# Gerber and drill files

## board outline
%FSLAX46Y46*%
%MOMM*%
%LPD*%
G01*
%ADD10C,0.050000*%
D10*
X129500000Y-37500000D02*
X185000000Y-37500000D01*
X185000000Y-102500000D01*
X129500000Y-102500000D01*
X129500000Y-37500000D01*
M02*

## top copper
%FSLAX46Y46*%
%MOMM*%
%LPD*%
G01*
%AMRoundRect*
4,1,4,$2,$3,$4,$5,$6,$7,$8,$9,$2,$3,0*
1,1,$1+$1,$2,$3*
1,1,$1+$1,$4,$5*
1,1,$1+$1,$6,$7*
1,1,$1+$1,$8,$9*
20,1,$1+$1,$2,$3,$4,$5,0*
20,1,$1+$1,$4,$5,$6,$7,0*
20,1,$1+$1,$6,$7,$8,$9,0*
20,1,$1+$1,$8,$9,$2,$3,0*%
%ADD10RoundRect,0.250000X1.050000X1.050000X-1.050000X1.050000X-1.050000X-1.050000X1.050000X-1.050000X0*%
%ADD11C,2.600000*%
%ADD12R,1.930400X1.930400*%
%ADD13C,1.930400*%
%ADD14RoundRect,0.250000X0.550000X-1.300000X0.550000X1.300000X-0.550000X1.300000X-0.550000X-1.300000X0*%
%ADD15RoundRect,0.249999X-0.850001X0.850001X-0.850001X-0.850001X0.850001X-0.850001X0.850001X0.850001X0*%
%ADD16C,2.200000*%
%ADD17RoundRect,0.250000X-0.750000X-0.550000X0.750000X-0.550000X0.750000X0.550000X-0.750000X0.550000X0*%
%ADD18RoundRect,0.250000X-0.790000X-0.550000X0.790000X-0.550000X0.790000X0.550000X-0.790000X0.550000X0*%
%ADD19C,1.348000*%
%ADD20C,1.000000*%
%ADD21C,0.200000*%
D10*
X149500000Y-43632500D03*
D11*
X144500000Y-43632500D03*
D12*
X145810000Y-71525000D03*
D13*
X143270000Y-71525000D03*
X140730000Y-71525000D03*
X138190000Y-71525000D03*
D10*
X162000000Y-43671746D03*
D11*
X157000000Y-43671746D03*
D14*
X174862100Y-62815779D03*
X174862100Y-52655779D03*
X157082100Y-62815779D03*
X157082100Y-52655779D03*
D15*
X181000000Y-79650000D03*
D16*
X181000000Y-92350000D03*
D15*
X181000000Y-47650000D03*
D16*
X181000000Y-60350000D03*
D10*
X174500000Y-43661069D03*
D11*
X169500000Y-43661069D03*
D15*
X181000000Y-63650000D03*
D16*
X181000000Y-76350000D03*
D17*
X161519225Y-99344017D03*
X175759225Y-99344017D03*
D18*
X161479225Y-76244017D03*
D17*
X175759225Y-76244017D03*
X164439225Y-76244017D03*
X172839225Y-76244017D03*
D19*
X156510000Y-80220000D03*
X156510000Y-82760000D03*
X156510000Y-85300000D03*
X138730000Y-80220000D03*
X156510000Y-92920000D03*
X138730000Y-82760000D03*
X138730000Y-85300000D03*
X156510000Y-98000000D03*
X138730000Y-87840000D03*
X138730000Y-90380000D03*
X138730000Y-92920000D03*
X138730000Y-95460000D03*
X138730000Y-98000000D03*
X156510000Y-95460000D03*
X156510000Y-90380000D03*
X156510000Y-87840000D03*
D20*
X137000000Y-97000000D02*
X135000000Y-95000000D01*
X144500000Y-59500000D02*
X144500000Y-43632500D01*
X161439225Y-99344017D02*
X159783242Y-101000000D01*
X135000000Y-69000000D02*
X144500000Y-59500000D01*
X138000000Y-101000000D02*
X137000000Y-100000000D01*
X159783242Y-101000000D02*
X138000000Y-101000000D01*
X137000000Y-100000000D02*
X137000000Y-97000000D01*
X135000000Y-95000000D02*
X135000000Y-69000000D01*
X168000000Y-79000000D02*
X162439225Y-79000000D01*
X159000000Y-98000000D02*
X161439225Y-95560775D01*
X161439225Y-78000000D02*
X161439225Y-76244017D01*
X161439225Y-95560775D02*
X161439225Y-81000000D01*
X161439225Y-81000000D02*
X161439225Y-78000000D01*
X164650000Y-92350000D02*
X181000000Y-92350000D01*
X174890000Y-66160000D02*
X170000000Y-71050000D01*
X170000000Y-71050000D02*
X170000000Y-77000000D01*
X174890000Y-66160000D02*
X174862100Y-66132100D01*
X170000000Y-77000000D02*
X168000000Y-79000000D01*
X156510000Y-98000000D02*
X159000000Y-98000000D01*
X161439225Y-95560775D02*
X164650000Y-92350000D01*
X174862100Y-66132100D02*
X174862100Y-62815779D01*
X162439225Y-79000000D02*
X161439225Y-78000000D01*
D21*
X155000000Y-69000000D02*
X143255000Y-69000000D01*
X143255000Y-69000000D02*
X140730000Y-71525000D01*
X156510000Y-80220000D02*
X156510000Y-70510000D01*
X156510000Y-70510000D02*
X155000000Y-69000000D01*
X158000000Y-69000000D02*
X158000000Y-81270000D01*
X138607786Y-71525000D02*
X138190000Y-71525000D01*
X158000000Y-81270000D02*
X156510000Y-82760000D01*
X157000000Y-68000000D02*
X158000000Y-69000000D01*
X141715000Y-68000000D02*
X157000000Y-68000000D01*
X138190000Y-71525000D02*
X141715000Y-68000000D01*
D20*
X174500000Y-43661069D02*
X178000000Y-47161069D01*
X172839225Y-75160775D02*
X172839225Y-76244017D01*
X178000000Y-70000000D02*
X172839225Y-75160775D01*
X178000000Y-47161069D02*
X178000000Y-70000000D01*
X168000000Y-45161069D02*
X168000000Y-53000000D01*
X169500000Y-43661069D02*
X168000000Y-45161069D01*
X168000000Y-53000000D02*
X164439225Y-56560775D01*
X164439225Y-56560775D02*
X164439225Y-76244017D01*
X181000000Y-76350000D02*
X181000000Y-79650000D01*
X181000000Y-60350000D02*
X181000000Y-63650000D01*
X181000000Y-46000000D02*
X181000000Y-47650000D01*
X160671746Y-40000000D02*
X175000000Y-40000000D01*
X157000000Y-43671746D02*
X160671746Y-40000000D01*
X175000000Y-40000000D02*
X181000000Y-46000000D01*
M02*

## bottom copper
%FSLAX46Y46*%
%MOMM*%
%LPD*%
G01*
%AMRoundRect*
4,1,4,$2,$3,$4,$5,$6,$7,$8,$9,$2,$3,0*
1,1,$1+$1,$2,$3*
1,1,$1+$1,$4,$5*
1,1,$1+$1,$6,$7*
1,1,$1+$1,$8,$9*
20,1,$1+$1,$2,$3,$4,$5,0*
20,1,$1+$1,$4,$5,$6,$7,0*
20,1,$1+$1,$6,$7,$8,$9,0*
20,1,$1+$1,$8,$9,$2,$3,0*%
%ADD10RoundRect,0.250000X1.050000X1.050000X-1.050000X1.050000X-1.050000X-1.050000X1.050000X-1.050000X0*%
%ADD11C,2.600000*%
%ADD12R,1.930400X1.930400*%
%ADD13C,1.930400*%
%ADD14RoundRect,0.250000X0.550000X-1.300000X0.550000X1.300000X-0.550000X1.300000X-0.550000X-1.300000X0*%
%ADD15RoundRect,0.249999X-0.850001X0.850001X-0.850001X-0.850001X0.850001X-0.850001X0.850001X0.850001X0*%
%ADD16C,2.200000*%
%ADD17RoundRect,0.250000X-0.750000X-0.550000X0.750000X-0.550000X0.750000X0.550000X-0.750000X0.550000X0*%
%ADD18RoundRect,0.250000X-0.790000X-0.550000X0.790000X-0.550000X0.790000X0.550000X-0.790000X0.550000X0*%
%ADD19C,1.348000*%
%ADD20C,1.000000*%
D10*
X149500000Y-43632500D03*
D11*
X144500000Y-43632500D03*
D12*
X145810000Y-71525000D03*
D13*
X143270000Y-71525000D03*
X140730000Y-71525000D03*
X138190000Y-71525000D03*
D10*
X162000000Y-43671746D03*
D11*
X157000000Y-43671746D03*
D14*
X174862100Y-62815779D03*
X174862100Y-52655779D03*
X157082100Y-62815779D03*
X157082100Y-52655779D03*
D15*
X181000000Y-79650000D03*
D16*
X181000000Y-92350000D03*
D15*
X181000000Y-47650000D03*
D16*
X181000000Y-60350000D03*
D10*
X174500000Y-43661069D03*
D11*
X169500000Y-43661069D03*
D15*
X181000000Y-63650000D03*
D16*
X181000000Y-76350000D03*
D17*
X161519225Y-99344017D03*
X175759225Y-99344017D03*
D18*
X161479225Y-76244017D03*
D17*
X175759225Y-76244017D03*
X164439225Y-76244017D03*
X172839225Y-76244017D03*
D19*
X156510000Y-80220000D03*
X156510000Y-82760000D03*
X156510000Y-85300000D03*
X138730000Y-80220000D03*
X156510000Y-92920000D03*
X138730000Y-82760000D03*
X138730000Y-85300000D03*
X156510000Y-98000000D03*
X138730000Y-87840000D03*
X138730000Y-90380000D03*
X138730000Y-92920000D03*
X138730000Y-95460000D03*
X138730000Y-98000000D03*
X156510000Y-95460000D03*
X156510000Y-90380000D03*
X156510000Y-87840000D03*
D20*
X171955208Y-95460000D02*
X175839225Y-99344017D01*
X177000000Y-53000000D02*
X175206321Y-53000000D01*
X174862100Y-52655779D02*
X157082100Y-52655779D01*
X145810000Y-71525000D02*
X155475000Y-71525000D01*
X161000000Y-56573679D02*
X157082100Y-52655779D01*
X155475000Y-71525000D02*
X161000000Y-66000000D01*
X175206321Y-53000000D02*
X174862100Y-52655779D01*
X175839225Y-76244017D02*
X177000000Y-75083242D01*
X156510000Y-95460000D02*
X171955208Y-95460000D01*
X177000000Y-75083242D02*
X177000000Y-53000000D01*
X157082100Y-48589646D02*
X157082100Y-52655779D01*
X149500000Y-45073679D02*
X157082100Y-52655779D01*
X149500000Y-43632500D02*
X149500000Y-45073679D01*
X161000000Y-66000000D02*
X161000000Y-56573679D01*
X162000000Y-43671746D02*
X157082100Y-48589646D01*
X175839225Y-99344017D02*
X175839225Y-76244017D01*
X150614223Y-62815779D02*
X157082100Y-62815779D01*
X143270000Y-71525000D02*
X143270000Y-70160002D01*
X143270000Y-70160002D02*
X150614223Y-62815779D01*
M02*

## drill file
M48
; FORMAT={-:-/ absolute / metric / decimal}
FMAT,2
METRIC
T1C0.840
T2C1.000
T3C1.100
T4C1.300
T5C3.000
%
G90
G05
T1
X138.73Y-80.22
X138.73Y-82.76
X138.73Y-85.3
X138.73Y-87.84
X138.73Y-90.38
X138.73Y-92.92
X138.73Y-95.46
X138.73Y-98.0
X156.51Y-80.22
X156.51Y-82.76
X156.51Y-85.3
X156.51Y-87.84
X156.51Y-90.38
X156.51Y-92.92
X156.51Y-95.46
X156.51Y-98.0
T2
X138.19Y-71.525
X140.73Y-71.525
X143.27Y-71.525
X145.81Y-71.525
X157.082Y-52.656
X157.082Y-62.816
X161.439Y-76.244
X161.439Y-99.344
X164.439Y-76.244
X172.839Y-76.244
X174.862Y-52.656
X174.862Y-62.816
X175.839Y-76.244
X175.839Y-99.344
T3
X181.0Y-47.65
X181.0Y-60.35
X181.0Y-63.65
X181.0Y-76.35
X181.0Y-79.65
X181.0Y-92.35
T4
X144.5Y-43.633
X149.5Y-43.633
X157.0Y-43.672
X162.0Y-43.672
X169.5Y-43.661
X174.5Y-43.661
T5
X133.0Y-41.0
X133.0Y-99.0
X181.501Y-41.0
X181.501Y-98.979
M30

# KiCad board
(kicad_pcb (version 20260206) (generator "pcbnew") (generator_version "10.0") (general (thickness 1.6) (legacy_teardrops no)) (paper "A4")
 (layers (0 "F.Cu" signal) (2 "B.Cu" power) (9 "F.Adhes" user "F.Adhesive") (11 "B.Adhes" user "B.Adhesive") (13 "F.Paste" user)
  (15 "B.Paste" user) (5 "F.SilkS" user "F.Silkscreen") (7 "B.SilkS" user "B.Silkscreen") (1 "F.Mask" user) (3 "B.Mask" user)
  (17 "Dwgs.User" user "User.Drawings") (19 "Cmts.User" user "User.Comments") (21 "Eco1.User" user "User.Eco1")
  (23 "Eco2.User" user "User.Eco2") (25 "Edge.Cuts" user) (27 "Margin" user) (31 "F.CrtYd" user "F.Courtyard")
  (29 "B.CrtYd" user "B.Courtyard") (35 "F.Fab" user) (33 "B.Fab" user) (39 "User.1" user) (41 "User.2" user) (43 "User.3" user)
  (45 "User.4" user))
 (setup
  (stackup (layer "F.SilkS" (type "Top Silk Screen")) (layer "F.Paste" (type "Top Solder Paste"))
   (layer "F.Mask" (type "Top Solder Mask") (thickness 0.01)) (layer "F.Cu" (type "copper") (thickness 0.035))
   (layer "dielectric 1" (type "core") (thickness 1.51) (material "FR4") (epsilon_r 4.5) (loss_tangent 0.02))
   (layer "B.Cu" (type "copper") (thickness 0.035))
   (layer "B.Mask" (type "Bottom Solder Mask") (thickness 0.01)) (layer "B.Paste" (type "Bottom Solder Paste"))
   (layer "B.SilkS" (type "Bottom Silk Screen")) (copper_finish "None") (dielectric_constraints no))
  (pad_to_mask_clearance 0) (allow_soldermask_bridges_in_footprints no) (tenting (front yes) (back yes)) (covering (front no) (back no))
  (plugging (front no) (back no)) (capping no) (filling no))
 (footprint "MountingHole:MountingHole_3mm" (layer "F.Cu") (at 133 99)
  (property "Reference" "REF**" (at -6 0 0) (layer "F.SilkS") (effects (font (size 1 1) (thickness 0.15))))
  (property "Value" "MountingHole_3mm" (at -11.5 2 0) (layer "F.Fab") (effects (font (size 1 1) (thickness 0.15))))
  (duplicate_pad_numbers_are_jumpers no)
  (pad "" np_thru_hole circle (at 0 0) (size 3 3) (drill 3) (layers "*.Cu" "*.Mask")))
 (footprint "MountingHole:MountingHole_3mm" (layer "F.Cu") (at 181.501076 41)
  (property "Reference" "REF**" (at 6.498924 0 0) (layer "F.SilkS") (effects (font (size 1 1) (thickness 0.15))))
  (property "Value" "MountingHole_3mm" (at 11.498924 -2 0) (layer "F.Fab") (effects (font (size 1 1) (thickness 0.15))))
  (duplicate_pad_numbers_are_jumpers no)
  (pad "" np_thru_hole circle (at 0 0) (size 3 3) (drill 3) (layers "*.Cu" "*.Mask")))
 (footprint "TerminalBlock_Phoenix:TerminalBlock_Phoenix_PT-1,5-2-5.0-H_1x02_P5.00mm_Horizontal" (layer "F.Cu") (at 149.5 43.6325 180)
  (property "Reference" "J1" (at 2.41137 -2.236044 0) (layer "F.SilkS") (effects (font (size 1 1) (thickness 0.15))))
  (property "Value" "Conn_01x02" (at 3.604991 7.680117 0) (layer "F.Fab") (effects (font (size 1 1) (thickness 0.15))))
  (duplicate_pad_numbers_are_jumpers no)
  (pad "1" thru_hole roundrect (at 0 0 180) (size 2.6 2.6) (drill 1.3) (layers "*.Cu" "*.Mask") (remove_unused_layers no)
   (roundrect_rratio 0.096154) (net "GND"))
  (pad "2" thru_hole circle (at 5 0 180) (size 2.6 2.6) (drill 1.3) (layers "*.Cu" "*.Mask") (remove_unused_layers no)
   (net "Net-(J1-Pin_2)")))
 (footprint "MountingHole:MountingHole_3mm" (layer "F.Cu") (at 181.501076 98.979038)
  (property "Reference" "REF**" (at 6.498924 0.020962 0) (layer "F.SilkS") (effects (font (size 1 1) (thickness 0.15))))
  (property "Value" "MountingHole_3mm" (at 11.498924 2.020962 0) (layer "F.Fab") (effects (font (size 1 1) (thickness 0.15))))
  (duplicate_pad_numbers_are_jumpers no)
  (pad "" np_thru_hole circle (at 0 0) (size 3 3) (drill 3) (layers "*.Cu" "*.Mask")))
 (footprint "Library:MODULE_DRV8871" (layer "F.Cu") (at 142 62)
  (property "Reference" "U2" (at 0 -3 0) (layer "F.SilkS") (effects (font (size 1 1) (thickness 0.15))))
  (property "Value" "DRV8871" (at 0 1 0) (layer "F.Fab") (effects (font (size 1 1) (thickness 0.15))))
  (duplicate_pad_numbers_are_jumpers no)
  (pad "1" thru_hole rect (at 3.81 9.525) (size 1.9304 1.9304) (drill 1) (layers "*.Cu" "*.Mask") (remove_unused_layers no) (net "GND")
   (solder_mask_margin 0.102))
  (pad "2" thru_hole circle (at 1.27 9.525) (size 1.9304 1.9304) (drill 1) (layers "*.Cu" "*.Mask") (remove_unused_layers no)
   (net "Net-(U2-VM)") (solder_mask_margin 0.102))
  (pad "3" thru_hole circle (at -1.27 9.525) (size 1.9304 1.9304) (drill 1) (layers "*.Cu" "*.Mask") (remove_unused_layers no)
   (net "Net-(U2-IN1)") (solder_mask_margin 0.102))
  (pad "4" thru_hole circle (at -3.81 9.525) (size 1.9304 1.9304) (drill 1) (layers "*.Cu" "*.Mask") (remove_unused_layers no)
   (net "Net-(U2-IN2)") (solder_mask_margin 0.102)))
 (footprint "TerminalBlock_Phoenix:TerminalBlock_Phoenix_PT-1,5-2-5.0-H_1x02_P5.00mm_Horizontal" (layer "F.Cu") (at 162 43.671746 180)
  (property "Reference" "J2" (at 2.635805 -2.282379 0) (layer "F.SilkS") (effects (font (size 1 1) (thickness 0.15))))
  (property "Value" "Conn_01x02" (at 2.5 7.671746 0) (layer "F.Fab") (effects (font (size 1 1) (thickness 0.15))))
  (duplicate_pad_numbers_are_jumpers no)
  (pad "1" thru_hole roundrect (at 0 0 180) (size 2.6 2.6) (drill 1.3) (layers "*.Cu" "*.Mask") (remove_unused_layers no)
   (roundrect_rratio 0.096154) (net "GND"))
  (pad "2" thru_hole circle (at 5 0 180) (size 2.6 2.6) (drill 1.3) (layers "*.Cu" "*.Mask") (remove_unused_layers no) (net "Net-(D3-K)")))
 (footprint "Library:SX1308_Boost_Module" (layer "F.Cu") (at 165.9721 57.735779 90)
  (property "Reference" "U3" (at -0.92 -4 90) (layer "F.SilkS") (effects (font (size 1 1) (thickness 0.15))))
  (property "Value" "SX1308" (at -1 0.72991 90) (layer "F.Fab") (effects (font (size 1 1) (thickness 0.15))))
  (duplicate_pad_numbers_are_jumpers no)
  (pad "1" thru_hole roundrect (at -5.08 8.89 90) (size 3.1 1.6) (drill 1) (layers "*.Cu" "*.Mask") (remove_unused_layers no)
   (roundrect_rratio 0.15625) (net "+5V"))
  (pad "2" thru_hole roundrect (at 5.08 8.89 90) (size 3.1 1.6) (drill 1) (layers "*.Cu" "*.Mask") (remove_unused_layers no)
   (roundrect_rratio 0.15625) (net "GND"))
  (pad "3" thru_hole roundrect (at -5.08 -8.89 90) (size 3.1 1.6) (drill 1) (layers "*.Cu" "*.Mask") (remove_unused_layers no)
   (roundrect_rratio 0.15625) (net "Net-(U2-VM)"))
  (pad "4" thru_hole roundrect (at 5.08 -8.89 90) (size 3.1 1.6) (drill 1) (layers "*.Cu" "*.Mask") (remove_unused_layers no)
   (roundrect_rratio 0.15625) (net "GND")))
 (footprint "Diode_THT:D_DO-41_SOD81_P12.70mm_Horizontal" (layer "F.Cu") (at 181 79.65 -90)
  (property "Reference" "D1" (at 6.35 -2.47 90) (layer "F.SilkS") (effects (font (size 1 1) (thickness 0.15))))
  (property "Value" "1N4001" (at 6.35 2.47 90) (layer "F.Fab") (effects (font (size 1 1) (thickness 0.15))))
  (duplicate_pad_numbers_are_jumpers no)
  (pad "1" thru_hole roundrect (at 0 0 270) (size 2.2 2.2) (drill 1.1) (layers "*.Cu" "*.Mask") (remove_unused_layers no)
   (roundrect_rratio 0.113636) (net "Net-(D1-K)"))
  (pad "2" thru_hole circle (at 12.7 0 270) (size 2.2 2.2) (drill 1.1) (layers "*.Cu" "*.Mask") (remove_unused_layers no) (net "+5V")))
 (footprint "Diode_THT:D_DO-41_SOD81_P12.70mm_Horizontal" (layer "F.Cu") (at 181 47.65 -90)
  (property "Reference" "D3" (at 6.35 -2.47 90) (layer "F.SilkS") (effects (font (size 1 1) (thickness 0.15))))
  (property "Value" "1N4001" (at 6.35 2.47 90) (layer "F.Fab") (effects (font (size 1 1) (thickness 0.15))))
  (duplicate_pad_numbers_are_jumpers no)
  (pad "1" thru_hole roundrect (at 0 0 270) (size 2.2 2.2) (drill 1.1) (layers "*.Cu" "*.Mask") (remove_unused_layers no)
   (roundrect_rratio 0.113636) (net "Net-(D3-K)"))
  (pad "2" thru_hole circle (at 12.7 0 270) (size 2.2 2.2) (drill 1.1) (layers "*.Cu" "*.Mask") (remove_unused_layers no) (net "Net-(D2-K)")))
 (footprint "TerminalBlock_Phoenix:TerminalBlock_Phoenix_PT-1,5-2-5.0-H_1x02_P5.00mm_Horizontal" (layer "F.Cu") (at 174.5 43.661069 180)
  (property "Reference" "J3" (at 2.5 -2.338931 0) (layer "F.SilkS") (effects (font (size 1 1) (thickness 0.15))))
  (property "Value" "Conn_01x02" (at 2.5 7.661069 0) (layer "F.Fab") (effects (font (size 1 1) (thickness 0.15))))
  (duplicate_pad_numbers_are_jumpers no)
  (pad "1" thru_hole roundrect (at 0 0 180) (size 2.6 2.6) (drill 1.3) (layers "*.Cu" "*.Mask") (remove_unused_layers no)
   (roundrect_rratio 0.096154) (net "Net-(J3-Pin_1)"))
  (pad "2" thru_hole circle (at 5 0 180) (size 2.6 2.6) (drill 1.3) (layers "*.Cu" "*.Mask") (remove_unused_layers no)
   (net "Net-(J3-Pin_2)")))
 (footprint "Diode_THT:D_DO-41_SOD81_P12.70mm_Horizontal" (layer "F.Cu") (at 181 63.65 -90)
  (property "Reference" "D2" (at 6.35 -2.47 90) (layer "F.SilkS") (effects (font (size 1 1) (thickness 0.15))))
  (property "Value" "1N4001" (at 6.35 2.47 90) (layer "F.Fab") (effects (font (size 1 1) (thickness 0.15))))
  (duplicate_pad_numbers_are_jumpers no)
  (pad "1" thru_hole roundrect (at 0 0 270) (size 2.2 2.2) (drill 1.1) (layers "*.Cu" "*.Mask") (remove_unused_layers no)
   (roundrect_rratio 0.113636) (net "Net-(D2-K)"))
  (pad "2" thru_hole circle (at 12.7 0 270) (size 2.2 2.2) (drill 1.1) (layers "*.Cu" "*.Mask") (remove_unused_layers no) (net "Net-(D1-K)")))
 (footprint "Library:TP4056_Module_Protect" (layer "F.Cu") (at 168.639225 86.894017)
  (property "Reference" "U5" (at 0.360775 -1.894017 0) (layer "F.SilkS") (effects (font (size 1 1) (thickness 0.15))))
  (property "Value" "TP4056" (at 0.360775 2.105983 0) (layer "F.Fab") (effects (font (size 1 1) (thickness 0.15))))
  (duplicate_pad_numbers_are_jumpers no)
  (pad "1" thru_hole roundrect (at -7.2 12.45) (size 2 1.6) (drill 1 (offset 0.08 0)) (layers "*.Cu" "*.Mask") (remove_unused_layers no)
   (roundrect_rratio 0.15625) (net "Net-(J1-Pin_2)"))
  (pad "2" thru_hole roundrect (at 7.2 12.45) (size 2 1.6) (drill 1 (offset -0.08 0)) (layers "*.Cu" "*.Mask") (remove_unused_layers no)
   (roundrect_rratio 0.15625) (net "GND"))
  (pad "3" thru_hole roundrect (at -7.2 -10.65) (size 2.08 1.6) (drill 1 (offset 0.04 0)) (layers "*.Cu" "*.Mask") (remove_unused_layers no)
   (roundrect_rratio 0.15625) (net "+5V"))
  (pad "4" thru_hole roundrect (at 7.2 -10.65) (size 2 1.6) (drill 1 (offset -0.08 0)) (layers "*.Cu" "*.Mask") (remove_unused_layers no)
   (roundrect_rratio 0.15625) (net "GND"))
  (pad "5" thru_hole roundrect (at -4.2 -10.65) (size 2 1.6) (drill 1) (layers "*.Cu" "*.Mask") (remove_unused_layers no)
   (roundrect_rratio 0.15625) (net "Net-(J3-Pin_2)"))
  (pad "6" thru_hole roundrect (at 4.2 -10.65) (size 2 1.6) (drill 1) (layers "*.Cu" "*.Mask") (remove_unused_layers no)
   (roundrect_rratio 0.15625) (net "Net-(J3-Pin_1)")))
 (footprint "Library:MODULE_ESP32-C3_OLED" (layer "F.Cu") (at 147.62 88.1 180)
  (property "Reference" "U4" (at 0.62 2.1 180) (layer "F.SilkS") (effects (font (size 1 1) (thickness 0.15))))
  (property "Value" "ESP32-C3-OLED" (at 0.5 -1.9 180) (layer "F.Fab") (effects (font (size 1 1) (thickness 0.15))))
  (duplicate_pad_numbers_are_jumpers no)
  (pad "0" thru_hole circle (at -8.89 7.88 180) (size 1.348 1.348) (drill 0.84) (layers "*.Cu" "*.Mask") (remove_unused_layers no)
   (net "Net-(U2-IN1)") (solder_mask_margin 0.102))
  (pad "1" thru_hole circle (at -8.89 5.34 180) (size 1.348 1.348) (drill 0.84) (layers "*.Cu" "*.Mask") (remove_unused_layers no)
   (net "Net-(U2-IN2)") (solder_mask_margin 0.102))
  (pad "2" thru_hole circle (at -8.89 2.8 180) (size 1.348 1.348) (drill 0.84) (layers "*.Cu" "*.Mask") (remove_unused_layers no)
   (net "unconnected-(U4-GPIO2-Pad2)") (solder_mask_margin 0.102))
  (pad "3" thru_hole circle (at 8.89 7.88 180) (size 1.348 1.348) (drill 0.84) (layers "*.Cu" "*.Mask") (remove_unused_layers no)
   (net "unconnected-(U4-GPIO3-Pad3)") (solder_mask_margin 0.102))
  (pad "3.3" thru_hole circle (at -8.89 -4.82 180) (size 1.348 1.348) (drill 0.84) (layers "*.Cu" "*.Mask") (remove_unused_layers no)
   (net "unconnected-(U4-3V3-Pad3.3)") (solder_mask_margin 0.102))
  (pad "4" thru_hole circle (at 8.89 5.34 180) (size 1.348 1.348) (drill 0.84) (layers "*.Cu" "*.Mask") (remove_unused_layers no)
   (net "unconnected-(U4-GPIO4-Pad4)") (solder_mask_margin 0.102))
  (pad "5" thru_hole circle (at 8.89 2.8 180) (size 1.348 1.348) (drill 0.84) (layers "*.Cu" "*.Mask") (remove_unused_layers no)
   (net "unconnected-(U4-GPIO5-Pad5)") (solder_mask_margin 0.102))
  (pad "5V" thru_hole circle (at -8.89 -9.9 180) (size 1.348 1.348) (drill 0.84) (layers "*.Cu" "*.Mask") (remove_unused_layers no)
   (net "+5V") (solder_mask_margin 0.102))
  (pad "6" thru_hole circle (at 8.89 0.26 180) (size 1.348 1.348) (drill 0.84) (layers "*.Cu" "*.Mask") (remove_unused_layers no)
   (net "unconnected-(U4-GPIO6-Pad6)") (solder_mask_margin 0.102))
  (pad "7" thru_hole circle (at 8.89 -2.28 180) (size 1.348 1.348) (drill 0.84) (layers "*.Cu" "*.Mask") (remove_unused_layers no)
   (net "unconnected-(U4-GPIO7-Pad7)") (solder_mask_margin 0.102))
  (pad "8" thru_hole circle (at 8.89 -4.82 180) (size 1.348 1.348) (drill 0.84) (layers "*.Cu" "*.Mask") (remove_unused_layers no)
   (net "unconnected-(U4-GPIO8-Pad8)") (solder_mask_margin 0.102))
  (pad "9" thru_hole circle (at 8.89 -7.36 180) (size 1.348 1.348) (drill 0.84) (layers "*.Cu" "*.Mask") (remove_unused_layers no)
   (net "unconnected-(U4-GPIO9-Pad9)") (solder_mask_margin 0.102))
  (pad "10" thru_hole circle (at 8.89 -9.9 180) (size 1.348 1.348) (drill 0.84) (layers "*.Cu" "*.Mask") (remove_unused_layers no)
   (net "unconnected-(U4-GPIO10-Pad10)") (solder_mask_margin 0.102))
  (pad "G" thru_hole circle (at -8.89 -7.36 180) (size 1.348 1.348) (drill 0.84) (layers "*.Cu" "*.Mask") (remove_unused_layers no)
   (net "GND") (solder_mask_margin 0.102))
  (pad "RX" thru_hole circle (at -8.89 -2.28 180) (size 1.348 1.348) (drill 0.84) (layers "*.Cu" "*.Mask") (remove_unused_layers no)
   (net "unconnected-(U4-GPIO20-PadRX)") (solder_mask_margin 0.102))
  (pad "TX" thru_hole circle (at -8.89 0.26 180) (size 1.348 1.348) (drill 0.84) (layers "*.Cu" "*.Mask") (remove_unused_layers no)
   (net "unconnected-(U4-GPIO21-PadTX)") (solder_mask_margin 0.102)))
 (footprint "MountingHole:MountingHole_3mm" (layer "F.Cu") (at 133 41)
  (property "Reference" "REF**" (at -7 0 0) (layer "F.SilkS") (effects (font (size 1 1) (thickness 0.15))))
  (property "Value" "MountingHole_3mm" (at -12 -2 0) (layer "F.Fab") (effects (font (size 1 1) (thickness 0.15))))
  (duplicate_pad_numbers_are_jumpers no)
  (pad "" np_thru_hole circle (at 0 0) (size 3 3) (drill 3) (layers "*.Cu" "*.Mask")))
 (gr_rect (start 129.5 37.5) (end 185 102.5) (stroke (width 0.05) (type default)) (fill no) (layer "Edge.Cuts"))
 (segment (start 137 97) (end 135 95) (width 1) (layer "F.Cu") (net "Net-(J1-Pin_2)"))
 (segment (start 144.5 59.5) (end 144.5 43.6325) (width 1) (layer "F.Cu") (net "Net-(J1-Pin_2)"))
 (segment (start 161.439225 99.344017) (end 159.783242 101) (width 1) (layer "F.Cu") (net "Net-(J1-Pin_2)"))
 (segment (start 135 69) (end 144.5 59.5) (width 1) (layer "F.Cu") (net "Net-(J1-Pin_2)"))
 (segment (start 138 101) (end 137 100) (width 1) (layer "F.Cu") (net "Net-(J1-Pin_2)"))
 (segment (start 159.783242 101) (end 138 101) (width 1) (layer "F.Cu") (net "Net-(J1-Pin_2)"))
 (segment (start 137 100) (end 137 97) (width 1) (layer "F.Cu") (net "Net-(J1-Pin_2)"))
 (segment (start 135 95) (end 135 69) (width 1) (layer "F.Cu") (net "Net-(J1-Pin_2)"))
 (segment (start 171.955208 95.46) (end 175.839225 99.344017) (width 1) (layer "B.Cu") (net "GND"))
 (segment (start 177 53) (end 175.206321 53) (width 1) (layer "B.Cu") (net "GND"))
 (segment (start 174.8621 52.655779) (end 157.0821 52.655779) (width 1) (layer "B.Cu") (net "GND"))
 (segment (start 145.81 71.525) (end 155.475 71.525) (width 1) (layer "B.Cu") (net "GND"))
 (segment (start 161 56.573679) (end 157.0821 52.655779) (width 1) (layer "B.Cu") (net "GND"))
 (segment (start 155.475 71.525) (end 161 66) (width 1) (layer "B.Cu") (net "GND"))
 (segment (start 175.206321 53) (end 174.8621 52.655779) (width 1) (layer "B.Cu") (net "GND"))
 (segment (start 175.839225 76.244017) (end 177 75.083242) (width 1) (layer "B.Cu") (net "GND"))
 (segment (start 156.51 95.46) (end 171.955208 95.46) (width 1) (layer "B.Cu") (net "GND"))
 (segment (start 177 75.083242) (end 177 53) (width 1) (layer "B.Cu") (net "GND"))
 (segment (start 157.0821 48.589646) (end 157.0821 52.655779) (width 1) (layer "B.Cu") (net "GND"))
 (segment (start 149.5 45.073679) (end 157.0821 52.655779) (width 1) (layer "B.Cu") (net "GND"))
 (segment (start 149.5 43.6325) (end 149.5 45.073679) (width 1) (layer "B.Cu") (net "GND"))
 (segment (start 161 66) (end 161 56.573679) (width 1) (layer "B.Cu") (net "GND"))
 (segment (start 162 43.671746) (end 157.0821 48.589646) (width 1) (layer "B.Cu") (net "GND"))
 (segment (start 175.839225 99.344017) (end 175.839225 76.244017) (width 1) (layer "B.Cu") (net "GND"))
 (segment (start 150.614223 62.815779) (end 157.0821 62.815779) (width 1) (layer "B.Cu") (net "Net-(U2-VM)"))
 (segment (start 143.27 71.525) (end 143.27 70.160002) (width 1) (layer "B.Cu") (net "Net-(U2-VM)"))
 (segment (start 143.27 70.160002) (end 150.614223 62.815779) (width 1) (layer "B.Cu") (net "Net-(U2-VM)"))
 (segment (start 168 79) (end 162.439225 79) (width 1) (layer "F.Cu") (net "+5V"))
 (segment (start 159 98) (end 161.439225 95.560775) (width 1) (layer "F.Cu") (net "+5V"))
 (segment (start 161.439225 78) (end 161.439225 76.244017) (width 1) (layer "F.Cu") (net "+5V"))
 (segment (start 161.439225 95.560775) (end 161.439225 81) (width 1) (layer "F.Cu") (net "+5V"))
 (segment (start 161.439225 81) (end 161.439225 78) (width 1) (layer "F.Cu") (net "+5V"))
 (segment (start 164.65 92.35) (end 181 92.35) (width 1) (layer "F.Cu") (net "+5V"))
 (segment (start 174.89 66.16) (end 170 71.05) (width 1) (layer "F.Cu") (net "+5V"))
 (segment (start 170 71.05) (end 170 77) (width 1) (layer "F.Cu") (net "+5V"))
 (segment (start 174.89 66.16) (end 174.8621 66.1321) (width 1) (layer "F.Cu") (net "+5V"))
 (segment (start 170 77) (end 168 79) (width 1) (layer "F.Cu") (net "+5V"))
 (segment (start 156.51 98) (end 159 98) (width 1) (layer "F.Cu") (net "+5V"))
 (segment (start 161.439225 95.560775) (end 164.65 92.35) (width 1) (layer "F.Cu") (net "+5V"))
 (segment (start 174.8621 66.1321) (end 174.8621 62.815779) (width 1) (layer "F.Cu") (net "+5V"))
 (segment (start 162.439225 79) (end 161.439225 78) (width 1) (layer "F.Cu") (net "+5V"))
 (segment (start 155 69) (end 143.255 69) (width 0.2) (layer "F.Cu") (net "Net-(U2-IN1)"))
 (segment (start 143.255 69) (end 140.73 71.525) (width 0.2) (layer "F.Cu") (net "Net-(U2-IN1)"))
 (segment (start 156.51 80.22) (end 156.51 70.51) (width 0.2) (layer "F.Cu") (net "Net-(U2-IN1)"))
 (segment (start 156.51 70.51) (end 155 69) (width 0.2) (layer "F.Cu") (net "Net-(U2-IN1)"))
 (segment (start 158 69) (end 158 81.27) (width 0.2) (layer "F.Cu") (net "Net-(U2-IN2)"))
 (segment (start 138.607786 71.525) (end 138.19 71.525) (width 0.2) (layer "F.Cu") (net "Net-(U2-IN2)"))
 (segment (start 158 81.27) (end 156.51 82.76) (width 0.2) (layer "F.Cu") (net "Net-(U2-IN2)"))
 (segment (start 157 68) (end 158 69) (width 0.2) (layer "F.Cu") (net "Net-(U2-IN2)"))
 (segment (start 141.715 68) (end 157 68) (width 0.2) (layer "F.Cu") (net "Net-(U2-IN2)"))
 (segment (start 138.19 71.525) (end 141.715 68) (width 0.2) (layer "F.Cu") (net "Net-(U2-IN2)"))
 (segment (start 174.5 43.661069) (end 178 47.161069) (width 1) (layer "F.Cu") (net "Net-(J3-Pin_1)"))
 (segment (start 172.839225 75.160775) (end 172.839225 76.244017) (width 1) (layer "F.Cu") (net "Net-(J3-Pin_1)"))
 (segment (start 178 70) (end 172.839225 75.160775) (width 1) (layer "F.Cu") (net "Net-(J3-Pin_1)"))
 (segment (start 178 47.161069) (end 178 70) (width 1) (layer "F.Cu") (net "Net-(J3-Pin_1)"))
 (segment (start 168 45.161069) (end 168 53) (width 1) (layer "F.Cu") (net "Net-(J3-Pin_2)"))
 (segment (start 169.5 43.661069) (end 168 45.161069) (width 1) (layer "F.Cu") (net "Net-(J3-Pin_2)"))
 (segment (start 168 53) (end 164.439225 56.560775) (width 1) (layer "F.Cu") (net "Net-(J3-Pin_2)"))
 (segment (start 164.439225 56.560775) (end 164.439225 76.244017) (width 1) (layer "F.Cu") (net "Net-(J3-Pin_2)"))
 (segment (start 181 76.35) (end 181 79.65) (width 1) (layer "F.Cu") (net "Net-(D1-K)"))
 (segment (start 181 60.35) (end 181 63.65) (width 1) (layer "F.Cu") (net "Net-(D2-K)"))
 (segment (start 181 46) (end 181 47.65) (width 1) (layer "F.Cu") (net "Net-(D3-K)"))
 (segment (start 160.671746 40) (end 175 40) (width 1) (layer "F.Cu") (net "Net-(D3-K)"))
 (segment (start 157 43.671746) (end 160.671746 40) (width 1) (layer "F.Cu") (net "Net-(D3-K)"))
 (segment (start 175 40) (end 181 46) (width 1) (layer "F.Cu") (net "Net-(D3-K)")))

